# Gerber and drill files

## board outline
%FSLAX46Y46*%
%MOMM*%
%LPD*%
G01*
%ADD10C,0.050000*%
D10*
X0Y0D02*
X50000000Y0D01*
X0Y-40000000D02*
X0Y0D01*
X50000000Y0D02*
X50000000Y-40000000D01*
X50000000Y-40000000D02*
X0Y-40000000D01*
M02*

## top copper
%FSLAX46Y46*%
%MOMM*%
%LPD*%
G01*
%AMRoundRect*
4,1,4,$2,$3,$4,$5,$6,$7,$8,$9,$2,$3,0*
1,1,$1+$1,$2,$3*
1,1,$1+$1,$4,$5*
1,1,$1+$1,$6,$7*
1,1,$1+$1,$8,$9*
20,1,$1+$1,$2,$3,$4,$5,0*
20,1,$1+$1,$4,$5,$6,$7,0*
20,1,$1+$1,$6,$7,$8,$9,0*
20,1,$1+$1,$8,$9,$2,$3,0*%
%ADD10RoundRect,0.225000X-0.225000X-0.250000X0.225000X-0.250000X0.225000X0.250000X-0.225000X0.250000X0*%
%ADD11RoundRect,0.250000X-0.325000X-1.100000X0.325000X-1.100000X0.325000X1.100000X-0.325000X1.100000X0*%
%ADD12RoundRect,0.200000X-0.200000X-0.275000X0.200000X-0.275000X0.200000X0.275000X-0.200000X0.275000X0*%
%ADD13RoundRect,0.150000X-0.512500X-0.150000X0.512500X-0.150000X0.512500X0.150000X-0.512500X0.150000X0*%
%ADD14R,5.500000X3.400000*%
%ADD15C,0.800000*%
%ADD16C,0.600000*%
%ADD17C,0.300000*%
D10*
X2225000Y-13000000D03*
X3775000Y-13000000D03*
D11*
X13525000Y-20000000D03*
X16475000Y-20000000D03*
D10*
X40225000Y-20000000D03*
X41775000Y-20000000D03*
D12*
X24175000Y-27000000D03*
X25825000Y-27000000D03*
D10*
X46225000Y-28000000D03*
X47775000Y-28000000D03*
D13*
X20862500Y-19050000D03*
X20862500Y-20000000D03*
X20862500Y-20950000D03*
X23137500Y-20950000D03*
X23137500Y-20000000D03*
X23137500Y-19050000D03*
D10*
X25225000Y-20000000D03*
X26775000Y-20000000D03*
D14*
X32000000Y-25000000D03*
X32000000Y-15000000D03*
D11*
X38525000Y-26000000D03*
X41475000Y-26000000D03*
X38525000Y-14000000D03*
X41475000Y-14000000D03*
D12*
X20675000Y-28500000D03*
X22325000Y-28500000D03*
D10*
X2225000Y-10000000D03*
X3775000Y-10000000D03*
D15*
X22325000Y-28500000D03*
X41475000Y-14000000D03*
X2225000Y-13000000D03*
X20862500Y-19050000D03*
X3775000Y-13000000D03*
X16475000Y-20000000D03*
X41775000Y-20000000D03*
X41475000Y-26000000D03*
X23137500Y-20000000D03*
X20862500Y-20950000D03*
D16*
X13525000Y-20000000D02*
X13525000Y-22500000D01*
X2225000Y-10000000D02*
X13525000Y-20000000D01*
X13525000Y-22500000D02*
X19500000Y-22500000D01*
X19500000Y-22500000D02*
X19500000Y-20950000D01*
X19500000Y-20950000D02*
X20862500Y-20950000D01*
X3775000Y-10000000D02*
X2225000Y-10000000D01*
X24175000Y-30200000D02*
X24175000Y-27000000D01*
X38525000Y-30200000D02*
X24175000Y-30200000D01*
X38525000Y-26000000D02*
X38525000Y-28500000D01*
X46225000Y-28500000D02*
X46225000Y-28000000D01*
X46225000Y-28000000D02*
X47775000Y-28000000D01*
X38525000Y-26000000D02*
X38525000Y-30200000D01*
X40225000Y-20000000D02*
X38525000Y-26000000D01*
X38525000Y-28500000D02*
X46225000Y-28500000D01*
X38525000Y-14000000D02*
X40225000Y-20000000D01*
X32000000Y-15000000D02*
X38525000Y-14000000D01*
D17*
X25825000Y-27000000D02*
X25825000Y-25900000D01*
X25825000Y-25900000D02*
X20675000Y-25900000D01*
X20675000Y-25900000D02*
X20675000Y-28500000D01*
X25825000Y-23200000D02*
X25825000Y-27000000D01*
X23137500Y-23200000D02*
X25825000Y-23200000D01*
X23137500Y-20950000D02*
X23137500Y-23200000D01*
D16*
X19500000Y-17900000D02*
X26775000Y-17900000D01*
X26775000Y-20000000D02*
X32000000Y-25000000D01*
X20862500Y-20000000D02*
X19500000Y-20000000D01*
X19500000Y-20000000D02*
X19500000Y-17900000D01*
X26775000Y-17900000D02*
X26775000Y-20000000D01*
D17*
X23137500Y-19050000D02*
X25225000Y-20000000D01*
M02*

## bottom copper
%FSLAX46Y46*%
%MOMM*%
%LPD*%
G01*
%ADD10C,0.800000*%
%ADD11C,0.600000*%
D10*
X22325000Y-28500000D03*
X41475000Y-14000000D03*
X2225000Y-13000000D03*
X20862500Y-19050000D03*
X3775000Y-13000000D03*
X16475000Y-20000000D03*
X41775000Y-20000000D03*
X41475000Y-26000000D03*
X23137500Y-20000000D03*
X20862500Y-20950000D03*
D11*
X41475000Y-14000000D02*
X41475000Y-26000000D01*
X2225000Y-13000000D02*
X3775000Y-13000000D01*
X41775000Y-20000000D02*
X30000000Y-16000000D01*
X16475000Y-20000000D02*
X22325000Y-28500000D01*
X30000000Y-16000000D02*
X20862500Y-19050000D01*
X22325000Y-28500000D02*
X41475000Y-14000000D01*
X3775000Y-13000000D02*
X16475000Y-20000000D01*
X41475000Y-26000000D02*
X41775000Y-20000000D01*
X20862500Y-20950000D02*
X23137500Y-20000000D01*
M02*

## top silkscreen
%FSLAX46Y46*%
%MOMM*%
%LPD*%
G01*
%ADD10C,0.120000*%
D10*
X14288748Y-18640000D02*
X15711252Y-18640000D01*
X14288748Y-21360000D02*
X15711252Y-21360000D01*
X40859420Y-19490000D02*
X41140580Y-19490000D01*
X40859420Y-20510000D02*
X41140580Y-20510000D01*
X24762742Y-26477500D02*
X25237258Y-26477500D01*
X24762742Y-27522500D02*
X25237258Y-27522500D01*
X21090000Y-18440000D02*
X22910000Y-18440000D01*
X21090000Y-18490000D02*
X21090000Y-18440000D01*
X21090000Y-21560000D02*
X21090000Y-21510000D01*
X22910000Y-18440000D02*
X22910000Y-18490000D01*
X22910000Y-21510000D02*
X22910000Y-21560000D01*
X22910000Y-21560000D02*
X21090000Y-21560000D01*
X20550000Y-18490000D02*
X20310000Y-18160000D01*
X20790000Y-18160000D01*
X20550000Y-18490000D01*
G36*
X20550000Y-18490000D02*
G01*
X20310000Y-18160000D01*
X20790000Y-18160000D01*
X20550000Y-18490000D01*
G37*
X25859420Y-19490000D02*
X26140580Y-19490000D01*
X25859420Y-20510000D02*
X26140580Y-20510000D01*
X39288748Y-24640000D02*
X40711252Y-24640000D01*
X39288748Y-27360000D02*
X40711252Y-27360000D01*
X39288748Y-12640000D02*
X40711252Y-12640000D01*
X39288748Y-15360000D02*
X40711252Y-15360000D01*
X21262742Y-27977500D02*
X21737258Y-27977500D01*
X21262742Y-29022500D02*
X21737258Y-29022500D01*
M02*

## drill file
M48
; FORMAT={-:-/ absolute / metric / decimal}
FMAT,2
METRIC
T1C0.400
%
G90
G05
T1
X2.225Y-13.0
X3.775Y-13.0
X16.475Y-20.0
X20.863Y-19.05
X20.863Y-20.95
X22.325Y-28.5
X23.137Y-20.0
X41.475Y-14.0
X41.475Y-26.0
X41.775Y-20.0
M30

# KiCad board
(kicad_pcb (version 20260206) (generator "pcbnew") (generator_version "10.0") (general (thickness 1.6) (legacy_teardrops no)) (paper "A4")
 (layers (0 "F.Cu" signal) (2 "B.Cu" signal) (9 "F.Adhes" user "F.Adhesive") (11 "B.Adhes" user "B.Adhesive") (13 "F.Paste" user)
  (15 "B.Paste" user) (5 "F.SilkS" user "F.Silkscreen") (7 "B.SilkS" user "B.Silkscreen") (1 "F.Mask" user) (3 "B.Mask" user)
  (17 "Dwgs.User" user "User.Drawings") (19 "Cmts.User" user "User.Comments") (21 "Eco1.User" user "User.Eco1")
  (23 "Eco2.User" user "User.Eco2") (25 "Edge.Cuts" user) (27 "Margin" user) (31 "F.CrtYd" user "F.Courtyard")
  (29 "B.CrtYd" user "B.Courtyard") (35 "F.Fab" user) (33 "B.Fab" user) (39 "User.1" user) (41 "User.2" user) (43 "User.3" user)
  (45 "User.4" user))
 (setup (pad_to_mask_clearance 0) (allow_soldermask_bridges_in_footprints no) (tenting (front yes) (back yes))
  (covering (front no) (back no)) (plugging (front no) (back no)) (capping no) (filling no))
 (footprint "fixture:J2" (layer "F.Cu") (at 3 13)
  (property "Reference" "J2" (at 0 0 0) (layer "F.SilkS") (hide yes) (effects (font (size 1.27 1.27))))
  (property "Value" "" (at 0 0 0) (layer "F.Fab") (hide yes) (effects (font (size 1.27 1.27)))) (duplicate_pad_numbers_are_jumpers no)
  (pad "1" smd roundrect (at -0.775 0) (size 0.9 0.95) (layers "F.Cu" "F.Mask" "F.Paste") (roundrect_rratio 0.25) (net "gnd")
   (thermal_bridge_angle 45))
  (pad "2" smd roundrect (at 0.775 0) (size 0.9 0.95) (layers "F.Cu" "F.Mask" "F.Paste") (roundrect_rratio 0.25) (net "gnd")
   (thermal_bridge_angle 45)))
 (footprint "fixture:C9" (layer "F.Cu") (at 15 20)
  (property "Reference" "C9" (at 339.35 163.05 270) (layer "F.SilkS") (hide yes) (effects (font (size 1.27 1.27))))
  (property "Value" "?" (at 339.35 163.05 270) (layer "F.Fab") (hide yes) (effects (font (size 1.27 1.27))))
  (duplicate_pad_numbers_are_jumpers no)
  (fp_line (start -0.711252 -1.36) (end 0.711252 -1.36) (stroke (width 0.12) (type solid)) (layer "F.SilkS"))
  (fp_line (start -0.711252 1.36) (end 0.711252 1.36) (stroke (width 0.12) (type solid)) (layer "F.SilkS"))
  (pad "1" smd roundrect (at -1.475 0) (size 1.15 2.7) (layers "F.Cu" "F.Mask" "F.Paste") (roundrect_rratio 0.217391) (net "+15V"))
  (pad "2" smd roundrect (at 1.475 0) (size 1.15 2.7) (layers "F.Cu" "F.Mask" "F.Paste") (roundrect_rratio 0.217391) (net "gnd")))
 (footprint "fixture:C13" (layer "F.Cu") (at 41 20)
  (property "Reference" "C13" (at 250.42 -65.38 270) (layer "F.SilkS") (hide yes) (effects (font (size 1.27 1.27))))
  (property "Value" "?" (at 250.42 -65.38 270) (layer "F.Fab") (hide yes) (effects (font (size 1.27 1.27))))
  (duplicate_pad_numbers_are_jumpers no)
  (fp_line (start -0.14058 -0.51) (end 0.14058 -0.51) (stroke (width 0.12) (type solid)) (layer "F.SilkS"))
  (fp_line (start -0.14058 0.51) (end 0.14058 0.51) (stroke (width 0.12) (type solid)) (layer "F.SilkS"))
  (pad "1" smd roundrect (at -0.775 0) (size 0.9 0.95) (layers "F.Cu" "F.Mask" "F.Paste") (roundrect_rratio 0.25) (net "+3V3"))
  (pad "2" smd roundrect (at 0.775 0) (size 0.9 0.95) (layers "F.Cu" "F.Mask" "F.Paste") (roundrect_rratio 0.25) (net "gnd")))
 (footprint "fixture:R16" (layer "F.Cu") (at 25 27)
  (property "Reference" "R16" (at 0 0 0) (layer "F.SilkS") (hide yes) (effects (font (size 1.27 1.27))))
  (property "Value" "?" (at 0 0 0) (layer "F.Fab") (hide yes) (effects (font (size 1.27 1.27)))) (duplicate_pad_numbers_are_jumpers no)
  (fp_line (start -0.237258 -0.5225) (end 0.237258 -0.5225) (stroke (width 0.12) (type solid)) (layer "F.SilkS"))
  (fp_line (start -0.237258 0.5225) (end 0.237258 0.5225) (stroke (width 0.12) (type solid)) (layer "F.SilkS"))
  (pad "1" smd roundrect (at -0.825 0) (size 0.8 0.95) (layers "F.Cu" "F.Mask" "F.Paste") (roundrect_rratio 0.25) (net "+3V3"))
  (pad "2" smd roundrect (at 0.825 0) (size 0.8 0.95) (layers "F.Cu" "F.Mask" "F.Paste") (roundrect_rratio 0.25) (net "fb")))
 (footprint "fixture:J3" (layer "F.Cu") (at 47 28)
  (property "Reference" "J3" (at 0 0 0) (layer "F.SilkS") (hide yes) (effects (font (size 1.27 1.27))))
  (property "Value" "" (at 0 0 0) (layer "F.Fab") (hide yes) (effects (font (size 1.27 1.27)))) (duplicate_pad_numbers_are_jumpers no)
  (pad "1" smd roundrect (at -0.775 0) (size 0.9 0.95) (layers "F.Cu" "F.Mask" "F.Paste") (roundrect_rratio 0.25) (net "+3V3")
   (thermal_bridge_angle 45))
  (pad "2" smd roundrect (at 0.775 0) (size 0.9 0.95) (layers "F.Cu" "F.Mask" "F.Paste") (roundrect_rratio 0.25) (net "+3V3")
   (thermal_bridge_angle 45)))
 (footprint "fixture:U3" (layer "F.Cu") (at 22 20)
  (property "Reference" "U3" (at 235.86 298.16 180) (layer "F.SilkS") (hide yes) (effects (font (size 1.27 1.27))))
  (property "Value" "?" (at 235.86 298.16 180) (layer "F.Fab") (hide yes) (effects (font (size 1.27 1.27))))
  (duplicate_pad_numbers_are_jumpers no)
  (fp_line (start -0.91 -1.56) (end 0.91 -1.56) (stroke (width 0.12) (type solid)) (layer "F.SilkS"))
  (fp_line (start -0.91 -1.51) (end -0.91 -1.56) (stroke (width 0.12) (type solid)) (layer "F.SilkS"))
  (fp_line (start -0.91 1.56) (end -0.91 1.51) (stroke (width 0.12) (type solid)) (layer "F.SilkS"))
  (fp_line (start 0.91 -1.56) (end 0.91 -1.51) (stroke (width 0.12) (type solid)) (layer "F.SilkS"))
  (fp_line (start 0.91 1.51) (end 0.91 1.56) (stroke (width 0.12) (type solid)) (layer "F.SilkS"))
  (fp_line (start 0.91 1.56) (end -0.91 1.56) (stroke (width 0.12) (type solid)) (layer "F.SilkS"))
  (fp_poly (pts (xy -1.45 -1.51) (xy -1.69 -1.84) (xy -1.21 -1.84)) (stroke (width 0.12) (type solid)) (fill yes) (layer "F.SilkS"))
  (pad "1" smd roundrect (at -1.1375 -0.95) (size 1.325 0.6) (layers "F.Cu" "F.Mask" "F.Paste") (roundrect_rratio 0.25) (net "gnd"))
  (pad "2" smd roundrect (at -1.1375 0) (size 1.325 0.6) (layers "F.Cu" "F.Mask" "F.Paste") (roundrect_rratio 0.25) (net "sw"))
  (pad "3" smd roundrect (at -1.1375 0.95) (size 1.325 0.6) (layers "F.Cu" "F.Mask" "F.Paste") (roundrect_rratio 0.25) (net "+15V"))
  (pad "4" smd roundrect (at 1.1375 0.95) (size 1.325 0.6) (layers "F.Cu" "F.Mask" "F.Paste") (roundrect_rratio 0.25) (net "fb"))
  (pad "5" smd roundrect (at 1.1375 0) (size 1.325 0.6) (layers "F.Cu" "F.Mask" "F.Paste") (roundrect_rratio 0.25) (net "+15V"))
  (pad "6" smd roundrect (at 1.1375 -0.95) (size 1.325 0.6) (layers "F.Cu" "F.Mask" "F.Paste") (roundrect_rratio 0.25) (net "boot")))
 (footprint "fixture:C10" (layer "F.Cu") (at 26 20)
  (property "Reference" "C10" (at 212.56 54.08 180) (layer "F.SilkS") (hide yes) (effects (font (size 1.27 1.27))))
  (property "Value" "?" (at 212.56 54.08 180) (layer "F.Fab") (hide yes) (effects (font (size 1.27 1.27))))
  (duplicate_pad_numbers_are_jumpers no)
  (fp_line (start -0.14058 -0.51) (end 0.14058 -0.51) (stroke (width 0.12) (type solid)) (layer "F.SilkS"))
  (fp_line (start -0.14058 0.51) (end 0.14058 0.51) (stroke (width 0.12) (type solid)) (layer "F.SilkS"))
  (pad "1" smd roundrect (at -0.775 0) (size 0.9 0.95) (layers "F.Cu" "F.Mask" "F.Paste") (roundrect_rratio 0.25) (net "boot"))
  (pad "2" smd roundrect (at 0.775 0) (size 0.9 0.95) (layers "F.Cu" "F.Mask" "F.Paste") (roundrect_rratio 0.25) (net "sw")))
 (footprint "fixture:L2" (layer "F.Cu") (at 32 20 90)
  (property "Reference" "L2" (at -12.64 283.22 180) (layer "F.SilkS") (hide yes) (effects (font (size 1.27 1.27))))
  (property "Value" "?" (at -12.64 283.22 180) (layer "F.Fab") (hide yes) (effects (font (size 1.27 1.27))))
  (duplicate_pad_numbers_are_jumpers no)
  (pad "1" smd rect (at -5 0 90) (size 3.4 5.5) (layers "F.Cu" "F.Mask" "F.Paste") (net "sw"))
  (pad "2" smd rect (at 5 0 90) (size 3.4 5.5) (layers "F.Cu" "F.Mask" "F.Paste") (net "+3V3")))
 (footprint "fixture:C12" (layer "F.Cu") (at 40 26)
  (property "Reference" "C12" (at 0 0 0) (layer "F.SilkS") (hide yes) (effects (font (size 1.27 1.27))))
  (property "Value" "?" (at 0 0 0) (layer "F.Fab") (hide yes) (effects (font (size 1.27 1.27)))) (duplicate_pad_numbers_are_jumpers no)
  (fp_line (start -0.711252 -1.36) (end 0.711252 -1.36) (stroke (width 0.12) (type solid)) (layer "F.SilkS"))
  (fp_line (start -0.711252 1.36) (end 0.711252 1.36) (stroke (width 0.12) (type solid)) (layer "F.SilkS"))
  (pad "1" smd roundrect (at -1.475 0) (size 1.15 2.7) (layers "F.Cu" "F.Mask" "F.Paste") (roundrect_rratio 0.217391) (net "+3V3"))
  (pad "2" smd roundrect (at 1.475 0) (size 1.15 2.7) (layers "F.Cu" "F.Mask" "F.Paste") (roundrect_rratio 0.217391) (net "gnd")))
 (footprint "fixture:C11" (layer "F.Cu") (at 40 14)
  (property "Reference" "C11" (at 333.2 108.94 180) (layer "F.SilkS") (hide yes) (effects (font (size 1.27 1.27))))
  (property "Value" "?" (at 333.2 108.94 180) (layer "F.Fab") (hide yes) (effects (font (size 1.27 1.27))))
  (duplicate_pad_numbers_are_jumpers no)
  (fp_line (start -0.711252 -1.36) (end 0.711252 -1.36) (stroke (width 0.12) (type solid)) (layer "F.SilkS"))
  (fp_line (start -0.711252 1.36) (end 0.711252 1.36) (stroke (width 0.12) (type solid)) (layer "F.SilkS"))
  (pad "1" smd roundrect (at -1.475 0) (size 1.15 2.7) (layers "F.Cu" "F.Mask" "F.Paste") (roundrect_rratio 0.217391) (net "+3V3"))
  (pad "2" smd roundrect (at 1.475 0) (size 1.15 2.7) (layers "F.Cu" "F.Mask" "F.Paste") (roundrect_rratio 0.217391) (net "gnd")))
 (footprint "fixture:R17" (layer "F.Cu") (at 21.5 28.5)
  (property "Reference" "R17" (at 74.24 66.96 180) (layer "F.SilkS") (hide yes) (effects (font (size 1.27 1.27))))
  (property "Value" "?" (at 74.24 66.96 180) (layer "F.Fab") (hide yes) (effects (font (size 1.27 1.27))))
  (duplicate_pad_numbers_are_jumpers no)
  (fp_line (start -0.237258 -0.5225) (end 0.237258 -0.5225) (stroke (width 0.12) (type solid)) (layer "F.SilkS"))
  (fp_line (start -0.237258 0.5225) (end 0.237258 0.5225) (stroke (width 0.12) (type solid)) (layer "F.SilkS"))
  (pad "1" smd roundrect (at -0.825 0) (size 0.8 0.95) (layers "F.Cu" "F.Mask" "F.Paste") (roundrect_rratio 0.25) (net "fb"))
  (pad "2" smd roundrect (at 0.825 0) (size 0.8 0.95) (layers "F.Cu" "F.Mask" "F.Paste") (roundrect_rratio 0.25) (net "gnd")))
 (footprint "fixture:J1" (layer "F.Cu") (at 3 10)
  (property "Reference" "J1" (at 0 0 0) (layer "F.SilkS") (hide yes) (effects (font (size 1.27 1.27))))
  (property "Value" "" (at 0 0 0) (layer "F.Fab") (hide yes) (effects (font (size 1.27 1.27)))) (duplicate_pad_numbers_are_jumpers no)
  (pad "1" smd roundrect (at -0.775 0) (size 0.9 0.95) (layers "F.Cu" "F.Mask" "F.Paste") (roundrect_rratio 0.25) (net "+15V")
   (thermal_bridge_angle 45))
  (pad "2" smd roundrect (at 0.775 0) (size 0.9 0.95) (layers "F.Cu" "F.Mask" "F.Paste") (roundrect_rratio 0.25) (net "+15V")
   (thermal_bridge_angle 45)))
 (gr_line (start 0 0) (end 50 0) (stroke (width 0.05) (type default)) (layer "Edge.Cuts"))
 (gr_line (start 0 40) (end 0 0) (stroke (width 0.05) (type default)) (layer "Edge.Cuts"))
 (gr_line (start 50 0) (end 50 40) (stroke (width 0.05) (type default)) (layer "Edge.Cuts"))
 (gr_line (start 50 40) (end 0 40) (stroke (width 0.05) (type default)) (layer "Edge.Cuts"))
 (via (at 22.325 28.5) (size 0.8) (drill 0.4) (layers "F.Cu" "B.Cu") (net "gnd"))
 (via (at 41.475 14) (size 0.8) (drill 0.4) (layers "F.Cu" "B.Cu") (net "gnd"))
 (via (at 2.225 13) (size 0.8) (drill 0.4) (layers "F.Cu" "B.Cu") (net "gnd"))
 (via (at 20.8625 19.05) (size 0.8) (drill 0.4) (layers "F.Cu" "B.Cu") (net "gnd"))
 (via (at 3.775 13) (size 0.8) (drill 0.4) (layers "F.Cu" "B.Cu") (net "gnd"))
 (via (at 16.475 20) (size 0.8) (drill 0.4) (layers "F.Cu" "B.Cu") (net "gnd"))
 (via (at 41.775 20) (size 0.8) (drill 0.4) (layers "F.Cu" "B.Cu") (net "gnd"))
 (via (at 41.475 26) (size 0.8) (drill 0.4) (layers "F.Cu" "B.Cu") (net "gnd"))
 (segment (start 41.475 14) (end 41.475 26) (width 0.6) (layer "B.Cu") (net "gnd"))
 (segment (start 2.225 13) (end 3.775 13) (width 0.6) (layer "B.Cu") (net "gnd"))
 (segment (start 41.775 20) (end 30 16) (width 0.6) (layer "B.Cu") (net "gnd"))
 (segment (start 16.475 20) (end 22.325 28.5) (width 0.6) (layer "B.Cu") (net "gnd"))
 (segment (start 30 16) (end 20.8625 19.05) (width 0.6) (layer "B.Cu") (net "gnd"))
 (segment (start 22.325 28.5) (end 41.475 14) (width 0.6) (layer "B.Cu") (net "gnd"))
 (segment (start 3.775 13) (end 16.475 20) (width 0.6) (layer "B.Cu") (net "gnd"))
 (segment (start 41.475 26) (end 41.775 20) (width 0.6) (layer "B.Cu") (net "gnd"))
 (segment (start 13.525 20) (end 13.525 22.5) (width 0.6) (layer "F.Cu") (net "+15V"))
 (segment (start 2.225 10) (end 13.525 20) (width 0.6) (layer "F.Cu") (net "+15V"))
 (segment (start 13.525 22.5) (end 19.5 22.5) (width 0.6) (layer "F.Cu") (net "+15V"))
 (segment (start 19.5 22.5) (end 19.5 20.95) (width 0.6) (layer "F.Cu") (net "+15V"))
 (segment (start 19.5 20.95) (end 20.8625 20.95) (width 0.6) (layer "F.Cu") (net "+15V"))
 (segment (start 3.775 10) (end 2.225 10) (width 0.6) (layer "F.Cu") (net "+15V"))
 (via (at 23.1375 20) (size 0.8) (drill 0.4) (layers "F.Cu" "B.Cu") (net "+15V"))
 (via (at 20.8625 20.95) (size 0.8) (drill 0.4) (layers "F.Cu" "B.Cu") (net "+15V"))
 (segment (start 20.8625 20.95) (end 23.1375 20) (width 0.6) (layer "B.Cu") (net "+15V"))
 (segment (start 24.175 30.2) (end 24.175 27) (width 0.6) (layer "F.Cu") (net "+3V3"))
 (segment (start 38.525 30.2) (end 24.175 30.2) (width 0.6) (layer "F.Cu") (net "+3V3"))
 (segment (start 38.525 26) (end 38.525 28.5) (width 0.6) (layer "F.Cu") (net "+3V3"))
 (segment (start 46.225 28.5) (end 46.225 28) (width 0.6) (layer "F.Cu") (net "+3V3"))
 (segment (start 46.225 28) (end 47.775 28) (width 0.6) (layer "F.Cu") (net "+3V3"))
 (segment (start 38.525 26) (end 38.525 30.2) (width 0.6) (layer "F.Cu") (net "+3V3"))
 (segment (start 40.225 20) (end 38.525 26) (width 0.6) (layer "F.Cu") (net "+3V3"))
 (segment (start 38.525 28.5) (end 46.225 28.5) (width 0.6) (layer "F.Cu") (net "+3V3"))
 (segment (start 38.525 14) (end 40.225 20) (width 0.6) (layer "F.Cu") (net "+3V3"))
 (segment (start 32 15) (end 38.525 14) (width 0.6) (layer "F.Cu") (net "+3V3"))
 (segment (start 25.825 27) (end 25.825 25.9) (width 0.3) (layer "F.Cu") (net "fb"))
 (segment (start 25.825 25.9) (end 20.675 25.9) (width 0.3) (layer "F.Cu") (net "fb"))
 (segment (start 20.675 25.9) (end 20.675 28.5) (width 0.3) (layer "F.Cu") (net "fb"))
 (segment (start 25.825 23.2) (end 25.825 27) (width 0.3) (layer "F.Cu") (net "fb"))
 (segment (start 23.1375 23.2) (end 25.825 23.2) (width 0.3) (layer "F.Cu") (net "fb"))
 (segment (start 23.1375 20.95) (end 23.1375 23.2) (width 0.3) (layer "F.Cu") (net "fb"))
 (segment (start 19.5 17.9) (end 26.775 17.9) (width 0.6) (layer "F.Cu") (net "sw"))
 (segment (start 26.775 20) (end 32 25) (width 0.6) (layer "F.Cu") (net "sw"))
 (segment (start 20.8625 20) (end 19.5 20) (width 0.6) (layer "F.Cu") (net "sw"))
 (segment (start 19.5 20) (end 19.5 17.9) (width 0.6) (layer "F.Cu") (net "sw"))
 (segment (start 26.775 17.9) (end 26.775 20) (width 0.6) (layer "F.Cu") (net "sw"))
 (segment (start 23.1375 19.05) (end 25.225 20) (width 0.3) (layer "F.Cu") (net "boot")))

